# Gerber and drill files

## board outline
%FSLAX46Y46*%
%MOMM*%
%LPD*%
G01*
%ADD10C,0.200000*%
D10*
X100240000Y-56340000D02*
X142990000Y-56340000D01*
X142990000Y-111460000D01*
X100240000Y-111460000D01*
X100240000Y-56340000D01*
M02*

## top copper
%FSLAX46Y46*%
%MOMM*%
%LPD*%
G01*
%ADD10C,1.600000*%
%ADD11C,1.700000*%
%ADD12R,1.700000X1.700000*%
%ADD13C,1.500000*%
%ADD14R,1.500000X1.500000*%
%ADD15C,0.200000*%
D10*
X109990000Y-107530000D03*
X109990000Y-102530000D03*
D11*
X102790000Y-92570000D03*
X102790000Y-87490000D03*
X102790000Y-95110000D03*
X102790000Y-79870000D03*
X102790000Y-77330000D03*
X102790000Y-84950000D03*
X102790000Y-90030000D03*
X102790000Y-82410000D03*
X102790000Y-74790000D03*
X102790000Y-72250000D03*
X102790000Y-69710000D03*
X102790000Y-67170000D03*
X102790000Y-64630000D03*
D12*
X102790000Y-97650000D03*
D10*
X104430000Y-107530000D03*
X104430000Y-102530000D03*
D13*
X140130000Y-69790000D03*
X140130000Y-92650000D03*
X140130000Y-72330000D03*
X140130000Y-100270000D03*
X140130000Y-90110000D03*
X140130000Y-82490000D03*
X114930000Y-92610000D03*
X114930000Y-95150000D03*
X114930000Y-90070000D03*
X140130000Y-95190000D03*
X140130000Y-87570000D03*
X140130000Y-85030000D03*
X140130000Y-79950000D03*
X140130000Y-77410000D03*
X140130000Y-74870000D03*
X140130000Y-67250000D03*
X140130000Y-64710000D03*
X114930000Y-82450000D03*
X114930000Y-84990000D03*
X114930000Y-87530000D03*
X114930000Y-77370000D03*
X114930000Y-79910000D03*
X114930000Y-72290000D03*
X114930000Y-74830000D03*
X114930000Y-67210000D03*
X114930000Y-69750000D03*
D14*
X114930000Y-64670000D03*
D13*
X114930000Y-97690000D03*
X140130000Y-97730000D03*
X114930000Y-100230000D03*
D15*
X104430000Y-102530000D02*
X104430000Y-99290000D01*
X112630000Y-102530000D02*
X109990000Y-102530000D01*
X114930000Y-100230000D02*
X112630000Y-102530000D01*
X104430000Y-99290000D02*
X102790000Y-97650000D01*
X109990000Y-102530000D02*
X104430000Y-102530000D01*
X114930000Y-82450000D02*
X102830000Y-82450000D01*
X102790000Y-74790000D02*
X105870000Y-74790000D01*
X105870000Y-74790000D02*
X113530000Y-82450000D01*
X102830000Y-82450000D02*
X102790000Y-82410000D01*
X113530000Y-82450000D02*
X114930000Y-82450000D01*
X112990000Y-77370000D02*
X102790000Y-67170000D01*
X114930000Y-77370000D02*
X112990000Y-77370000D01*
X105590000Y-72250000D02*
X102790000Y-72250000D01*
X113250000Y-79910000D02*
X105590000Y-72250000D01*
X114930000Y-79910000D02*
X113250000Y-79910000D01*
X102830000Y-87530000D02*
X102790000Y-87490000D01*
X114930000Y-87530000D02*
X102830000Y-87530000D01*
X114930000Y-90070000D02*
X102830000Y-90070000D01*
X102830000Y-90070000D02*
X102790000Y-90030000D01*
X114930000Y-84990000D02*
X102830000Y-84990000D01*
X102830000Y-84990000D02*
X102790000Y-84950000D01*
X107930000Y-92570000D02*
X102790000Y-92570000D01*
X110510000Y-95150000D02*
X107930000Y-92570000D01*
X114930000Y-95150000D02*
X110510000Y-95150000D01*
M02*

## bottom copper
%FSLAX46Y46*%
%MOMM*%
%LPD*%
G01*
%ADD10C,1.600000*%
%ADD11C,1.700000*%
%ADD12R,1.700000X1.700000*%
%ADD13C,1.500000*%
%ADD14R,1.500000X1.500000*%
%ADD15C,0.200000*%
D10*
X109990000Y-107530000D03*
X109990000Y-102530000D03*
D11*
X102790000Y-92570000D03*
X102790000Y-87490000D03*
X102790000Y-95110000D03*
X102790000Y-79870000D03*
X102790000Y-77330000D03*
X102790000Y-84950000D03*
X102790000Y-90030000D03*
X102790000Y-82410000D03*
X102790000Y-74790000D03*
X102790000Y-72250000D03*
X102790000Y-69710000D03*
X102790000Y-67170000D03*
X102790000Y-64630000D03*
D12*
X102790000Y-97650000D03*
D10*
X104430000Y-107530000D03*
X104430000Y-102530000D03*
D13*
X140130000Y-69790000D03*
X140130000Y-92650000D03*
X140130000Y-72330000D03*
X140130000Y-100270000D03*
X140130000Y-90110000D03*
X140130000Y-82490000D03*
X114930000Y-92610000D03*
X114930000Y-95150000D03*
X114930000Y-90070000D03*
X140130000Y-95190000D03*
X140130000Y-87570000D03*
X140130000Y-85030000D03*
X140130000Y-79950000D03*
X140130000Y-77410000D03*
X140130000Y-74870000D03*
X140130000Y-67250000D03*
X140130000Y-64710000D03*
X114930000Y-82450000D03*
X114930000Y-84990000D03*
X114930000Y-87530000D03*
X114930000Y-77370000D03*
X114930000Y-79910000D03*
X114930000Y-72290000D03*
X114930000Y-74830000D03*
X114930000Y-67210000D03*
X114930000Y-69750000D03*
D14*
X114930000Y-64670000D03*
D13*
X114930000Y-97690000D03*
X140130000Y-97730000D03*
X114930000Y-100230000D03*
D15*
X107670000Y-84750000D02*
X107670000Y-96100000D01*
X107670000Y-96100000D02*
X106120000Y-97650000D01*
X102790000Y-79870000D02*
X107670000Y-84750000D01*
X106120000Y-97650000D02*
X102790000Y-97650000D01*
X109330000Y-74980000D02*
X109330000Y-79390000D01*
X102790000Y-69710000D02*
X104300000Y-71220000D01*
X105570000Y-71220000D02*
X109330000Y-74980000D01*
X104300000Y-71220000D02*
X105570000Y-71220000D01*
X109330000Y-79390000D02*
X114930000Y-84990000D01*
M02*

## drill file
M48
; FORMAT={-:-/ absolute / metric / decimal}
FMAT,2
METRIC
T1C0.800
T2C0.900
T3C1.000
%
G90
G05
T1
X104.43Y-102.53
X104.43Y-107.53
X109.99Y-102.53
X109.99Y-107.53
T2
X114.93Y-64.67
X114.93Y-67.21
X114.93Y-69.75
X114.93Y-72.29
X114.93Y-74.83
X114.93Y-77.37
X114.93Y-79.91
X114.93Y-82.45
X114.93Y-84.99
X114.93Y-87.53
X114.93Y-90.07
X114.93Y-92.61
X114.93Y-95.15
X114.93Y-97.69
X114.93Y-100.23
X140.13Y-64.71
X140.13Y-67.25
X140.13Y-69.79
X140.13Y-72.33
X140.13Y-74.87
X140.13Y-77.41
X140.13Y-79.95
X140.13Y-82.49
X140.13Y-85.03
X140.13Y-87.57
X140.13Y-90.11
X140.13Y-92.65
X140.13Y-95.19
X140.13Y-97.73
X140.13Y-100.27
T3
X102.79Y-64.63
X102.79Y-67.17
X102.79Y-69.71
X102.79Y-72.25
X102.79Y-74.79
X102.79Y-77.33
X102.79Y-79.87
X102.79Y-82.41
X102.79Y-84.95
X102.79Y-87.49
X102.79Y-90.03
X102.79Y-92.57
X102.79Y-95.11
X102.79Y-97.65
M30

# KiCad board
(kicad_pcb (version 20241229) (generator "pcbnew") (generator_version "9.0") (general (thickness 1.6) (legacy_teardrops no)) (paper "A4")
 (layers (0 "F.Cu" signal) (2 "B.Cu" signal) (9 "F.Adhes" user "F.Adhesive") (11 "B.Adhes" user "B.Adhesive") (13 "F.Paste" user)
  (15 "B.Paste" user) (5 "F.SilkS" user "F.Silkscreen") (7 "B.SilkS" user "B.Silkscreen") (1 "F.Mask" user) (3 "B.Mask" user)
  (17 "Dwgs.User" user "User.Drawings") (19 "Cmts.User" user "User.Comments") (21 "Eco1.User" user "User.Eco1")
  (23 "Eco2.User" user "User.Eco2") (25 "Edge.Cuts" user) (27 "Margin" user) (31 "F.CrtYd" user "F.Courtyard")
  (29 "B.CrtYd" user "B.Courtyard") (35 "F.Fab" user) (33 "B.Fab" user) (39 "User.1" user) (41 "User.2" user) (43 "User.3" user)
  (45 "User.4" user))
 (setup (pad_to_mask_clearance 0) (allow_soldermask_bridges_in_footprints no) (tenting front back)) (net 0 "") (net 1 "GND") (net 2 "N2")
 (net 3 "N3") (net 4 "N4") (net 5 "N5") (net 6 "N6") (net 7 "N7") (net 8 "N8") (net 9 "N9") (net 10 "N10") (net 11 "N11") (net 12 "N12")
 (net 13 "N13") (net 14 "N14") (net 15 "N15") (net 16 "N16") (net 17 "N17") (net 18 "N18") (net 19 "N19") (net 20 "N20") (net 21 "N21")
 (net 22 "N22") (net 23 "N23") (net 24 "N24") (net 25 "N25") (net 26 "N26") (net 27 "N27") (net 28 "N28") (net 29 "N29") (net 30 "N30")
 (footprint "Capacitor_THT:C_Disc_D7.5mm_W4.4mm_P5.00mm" (layer "F.Cu") (at 109.99 107.53 90)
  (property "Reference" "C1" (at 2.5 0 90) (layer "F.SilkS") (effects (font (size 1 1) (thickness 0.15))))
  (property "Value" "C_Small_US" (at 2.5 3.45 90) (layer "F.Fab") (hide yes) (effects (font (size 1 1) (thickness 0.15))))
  (pad "1" thru_hole circle (at 0 0 90) (size 1.6 1.6) (drill 0.8) (layers "*.Cu" "*.Mask") (remove_unused_layers no) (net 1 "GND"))
  (pad "2" thru_hole circle (at 5 0 90) (size 1.6 1.6) (drill 0.8) (layers "*.Cu" "*.Mask") (remove_unused_layers no) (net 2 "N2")))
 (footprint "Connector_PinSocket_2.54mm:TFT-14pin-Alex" (layer "F.Cu") (at 102.79 97.65 180)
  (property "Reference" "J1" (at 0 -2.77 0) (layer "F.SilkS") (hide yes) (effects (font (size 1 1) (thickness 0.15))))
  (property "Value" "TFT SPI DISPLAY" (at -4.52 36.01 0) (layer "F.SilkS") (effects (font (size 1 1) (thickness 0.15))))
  (pad "CS" thru_hole circle (at 0 5.08 180) (size 1.7 1.7) (drill 1) (layers "*.Cu" "*.Mask") (remove_unused_layers no) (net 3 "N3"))
  (pad "DC" thru_hole circle (at 0 10.16 180) (size 1.7 1.7) (drill 1) (layers "*.Cu" "*.Mask") (remove_unused_layers no) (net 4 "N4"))
  (pad "GND" thru_hole circle (at 0 2.54 180) (size 1.7 1.7) (drill 1) (layers "*.Cu" "*.Mask") (remove_unused_layers no) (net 1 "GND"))
  (pad "LED" thru_hole circle (at 0 17.78 180) (size 1.7 1.7) (drill 1) (layers "*.Cu" "*.Mask") (remove_unused_layers no) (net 2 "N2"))
  (pad "MISO" thru_hole circle (at 0 20.32 180) (size 1.7 1.7) (drill 1) (layers "*.Cu" "*.Mask") (remove_unused_layers no) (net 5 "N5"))
  (pad "MOSI" thru_hole circle (at 0 12.7 180) (size 1.7 1.7) (drill 1) (layers "*.Cu" "*.Mask") (remove_unused_layers no) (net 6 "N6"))
  (pad "RST" thru_hole circle (at 0 7.62 180) (size 1.7 1.7) (drill 1) (layers "*.Cu" "*.Mask") (remove_unused_layers no) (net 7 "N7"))
  (pad "SCK" thru_hole circle (at 0 15.24 180) (size 1.7 1.7) (drill 1) (layers "*.Cu" "*.Mask") (remove_unused_layers no) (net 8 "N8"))
  (pad "T_CLK" thru_hole circle (at 0 22.86 180) (size 1.7 1.7) (drill 1) (layers "*.Cu" "*.Mask") (remove_unused_layers no) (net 8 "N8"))
  (pad "T_CS" thru_hole circle (at 0 25.4 180) (size 1.7 1.7) (drill 1) (layers "*.Cu" "*.Mask") (remove_unused_layers no) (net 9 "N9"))
  (pad "T_DIN" thru_hole circle (at 0 27.94 180) (size 1.7 1.7) (drill 1) (layers "*.Cu" "*.Mask") (remove_unused_layers no) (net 6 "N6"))
  (pad "T_DO" thru_hole circle (at 0 30.48 180) (size 1.7 1.7) (drill 1) (layers "*.Cu" "*.Mask") (remove_unused_layers no) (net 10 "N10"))
  (pad "T_IRQ" thru_hole circle (at 0 33.02 180) (size 1.7 1.7) (drill 1) (layers "*.Cu" "*.Mask") (remove_unused_layers no) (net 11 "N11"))
  (pad "VCC" thru_hole rect (at 0 0 180) (size 1.7 1.7) (drill 1) (layers "*.Cu" "*.Mask") (remove_unused_layers no) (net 2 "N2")))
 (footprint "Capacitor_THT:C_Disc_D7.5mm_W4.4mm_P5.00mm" (layer "F.Cu") (at 104.43 107.53 90)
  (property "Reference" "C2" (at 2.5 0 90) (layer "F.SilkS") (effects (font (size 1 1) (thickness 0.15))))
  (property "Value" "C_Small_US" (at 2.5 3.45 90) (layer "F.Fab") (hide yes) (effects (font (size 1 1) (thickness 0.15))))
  (pad "1" thru_hole circle (at 0 0 90) (size 1.6 1.6) (drill 0.8) (layers "*.Cu" "*.Mask") (remove_unused_layers no) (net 1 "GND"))
  (pad "2" thru_hole circle (at 5 0 90) (size 1.6 1.6) (drill 0.8) (layers "*.Cu" "*.Mask") (remove_unused_layers no) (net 2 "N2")))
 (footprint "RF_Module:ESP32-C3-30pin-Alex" (layer "F.Cu") (at 114.93 64.67)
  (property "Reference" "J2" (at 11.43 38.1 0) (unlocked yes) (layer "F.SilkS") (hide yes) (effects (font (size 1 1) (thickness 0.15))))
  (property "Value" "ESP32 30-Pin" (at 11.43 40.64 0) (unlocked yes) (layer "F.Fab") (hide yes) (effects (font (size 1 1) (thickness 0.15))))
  (pad "1" thru_hole circle (at 25.2 5.12) (size 1.5 1.5) (drill 0.9) (layers "*.Cu" "*.Mask") (remove_unused_layers yes)
   (keep_end_layers yes) (zone_layer_connections) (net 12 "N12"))
  (pad "2" thru_hole circle (at 25.2 27.98) (size 1.5 1.5) (drill 0.9) (layers "*.Cu" "*.Mask") (remove_unused_layers yes)
   (keep_end_layers yes) (zone_layer_connections) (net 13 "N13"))
  (pad "3" thru_hole circle (at 25.2 7.66) (size 1.5 1.5) (drill 0.9) (layers "*.Cu" "*.Mask") (remove_unused_layers yes)
   (keep_end_layers yes) (zone_layer_connections) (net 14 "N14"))
  (pad "3.3V" thru_hole circle (at 25.2 35.6) (size 1.5 1.5) (drill 0.9) (layers "*.Cu" "*.Mask") (remove_unused_layers yes)
   (keep_end_layers yes) (zone_layer_connections))
  (pad "4" thru_hole circle (at 25.2 25.44) (size 1.5 1.5) (drill 0.9) (layers "*.Cu" "*.Mask") (remove_unused_layers yes)
   (keep_end_layers yes) (zone_layer_connections) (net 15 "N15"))
  (pad "5" thru_hole circle (at 25.2 17.82) (size 1.5 1.5) (drill 0.9) (layers "*.Cu" "*.Mask") (remove_unused_layers yes)
   (keep_end_layers yes) (zone_layer_connections) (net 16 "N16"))
  (pad "12" thru_hole circle (at 0 27.94) (size 1.5 1.5) (drill 0.9) (layers "*.Cu" "*.Mask") (remove_unused_layers yes)
   (keep_end_layers yes) (zone_layer_connections) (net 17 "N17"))
  (pad "13" thru_hole circle (at 0 30.48) (size 1.5 1.5) (drill 0.9) (layers "*.Cu" "*.Mask") (remove_unused_layers yes)
   (keep_end_layers yes) (zone_layer_connections) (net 3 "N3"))
  (pad "14" thru_hole circle (at 0 25.4) (size 1.5 1.5) (drill 0.9) (layers "*.Cu" "*.Mask") (remove_unused_layers yes)
   (keep_end_layers yes) (zone_layer_connections) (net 7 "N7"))
  (pad "15" thru_hole circle (at 25.2 30.52) (size 1.5 1.5) (drill 0.9) (layers "*.Cu" "*.Mask") (remove_unused_layers yes)
   (keep_end_layers yes) (zone_layer_connections) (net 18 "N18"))
  (pad "16" thru_hole circle (at 25.2 22.9) (size 1.5 1.5) (drill 0.9) (layers "*.Cu" "*.Mask") (remove_unused_layers yes)
   (keep_end_layers yes) (zone_layer_connections) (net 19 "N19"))
  (pad "17" thru_hole circle (at 25.2 20.36) (size 1.5 1.5) (drill 0.9) (layers "*.Cu" "*.Mask") (remove_unused_layers yes)
   (keep_end_layers yes) (zone_layer_connections) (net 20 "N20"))
  (pad "18" thru_hole circle (at 25.2 15.28) (size 1.5 1.5) (drill 0.9) (layers "*.Cu" "*.Mask") (remove_unused_layers yes)
   (keep_end_layers yes) (zone_layer_connections) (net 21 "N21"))
  (pad "19" thru_hole circle (at 25.2 12.74) (size 1.5 1.5) (drill 0.9) (layers "*.Cu" "*.Mask") (remove_unused_layers yes)
   (keep_end_layers yes) (zone_layer_connections) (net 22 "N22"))
  (pad "21" thru_hole circle (at 25.2 10.2) (size 1.5 1.5) (drill 0.9) (layers "*.Cu" "*.Mask") (remove_unused_layers yes)
   (keep_end_layers yes) (zone_layer_connections) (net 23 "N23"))
  (pad "22" thru_hole circle (at 25.2 2.58) (size 1.5 1.5) (drill 0.9) (layers "*.Cu" "*.Mask") (remove_unused_layers yes)
   (keep_end_layers yes) (zone_layer_connections) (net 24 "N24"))
  (pad "23" thru_hole circle (at 25.2 0.04) (size 1.5 1.5) (drill 0.9) (layers "*.Cu" "*.Mask") (remove_unused_layers yes)
   (keep_end_layers yes) (zone_layer_connections) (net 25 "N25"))
  (pad "25" thru_hole circle (at 0 17.78) (size 1.5 1.5) (drill 0.9) (layers "*.Cu" "*.Mask") (remove_unused_layers yes)
   (keep_end_layers yes) (zone_layer_connections) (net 8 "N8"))
  (pad "26" thru_hole circle (at 0 20.32) (size 1.5 1.5) (drill 0.9) (layers "*.Cu" "*.Mask") (remove_unused_layers yes)
   (keep_end_layers yes) (zone_layer_connections) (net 6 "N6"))
  (pad "27" thru_hole circle (at 0 22.86) (size 1.5 1.5) (drill 0.9) (layers "*.Cu" "*.Mask") (remove_unused_layers yes)
   (keep_end_layers yes) (zone_layer_connections) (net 4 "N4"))
  (pad "32" thru_hole circle (at 0 12.7) (size 1.5 1.5) (drill 0.9) (layers "*.Cu" "*.Mask") (remove_unused_layers yes)
   (keep_end_layers yes) (zone_layer_connections) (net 10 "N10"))
  (pad "33" thru_hole circle (at 0 15.24) (size 1.5 1.5) (drill 0.9) (layers "*.Cu" "*.Mask") (remove_unused_layers yes)
   (keep_end_layers yes) (zone_layer_connections) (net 9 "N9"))
  (pad "34" thru_hole circle (at 0 7.62) (size 1.5 1.5) (drill 0.9) (layers "*.Cu" "*.Mask") (remove_unused_layers yes)
   (keep_end_layers yes) (zone_layer_connections) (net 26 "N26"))
  (pad "35" thru_hole circle (at 0 10.16) (size 1.5 1.5) (drill 0.9) (layers "*.Cu" "*.Mask") (remove_unused_layers yes)
   (keep_end_layers yes) (zone_layer_connections) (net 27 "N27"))
  (pad "36" thru_hole circle (at 0 2.54) (size 1.5 1.5) (drill 0.9) (layers "*.Cu" "*.Mask") (remove_unused_layers yes)
   (keep_end_layers yes) (zone_layer_connections) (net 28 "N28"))
  (pad "39" thru_hole circle (at 0 5.08) (size 1.5 1.5) (drill 0.9) (layers "*.Cu" "*.Mask") (remove_unused_layers yes)
   (keep_end_layers yes) (zone_layer_connections) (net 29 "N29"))
  (pad "EN" thru_hole rect (at 0 0) (size 1.5 1.5) (drill 0.9) (layers "*.Cu" "*.Mask") (remove_unused_layers yes) (keep_end_layers yes)
   (zone_layer_connections) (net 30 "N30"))
  (pad "GND" thru_hole circle (at 0 33.02) (size 1.5 1.5) (drill 0.9) (layers "*.Cu" "*.Mask") (remove_unused_layers yes)
   (keep_end_layers yes) (zone_layer_connections) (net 1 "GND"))
  (pad "GND" thru_hole circle (at 25.2 33.06) (size 1.5 1.5) (drill 0.9) (layers "*.Cu" "*.Mask") (remove_unused_layers yes)
   (keep_end_layers yes) (zone_layer_connections) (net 1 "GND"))
  (pad "VIN" thru_hole circle (at 0 35.56) (size 1.5 1.5) (drill 0.9) (layers "*.Cu" "*.Mask") (remove_unused_layers yes)
   (keep_end_layers yes) (zone_layer_connections) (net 2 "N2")))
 (gr_rect (start 100.24 56.34) (end 142.99 111.46) (stroke (width 0.2) (type solid)) (fill no) (layer "Edge.Cuts"))
 (segment (start 104.43 102.53) (end 104.43 99.29) (width 0.2) (layer "F.Cu") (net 2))
 (segment (start 112.63 102.53) (end 109.99 102.53) (width 0.2) (layer "F.Cu") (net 2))
 (segment (start 114.93 100.23) (end 112.63 102.53) (width 0.2) (layer "F.Cu") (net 2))
 (segment (start 104.43 99.29) (end 102.79 97.65) (width 0.2) (layer "F.Cu") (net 2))
 (segment (start 109.99 102.53) (end 104.43 102.53) (width 0.2) (layer "F.Cu") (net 2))
 (segment (start 107.67 84.75) (end 107.67 96.1) (width 0.2) (layer "B.Cu") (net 2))
 (segment (start 107.67 96.1) (end 106.12 97.65) (width 0.2) (layer "B.Cu") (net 2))
 (segment (start 102.79 79.87) (end 107.67 84.75) (width 0.2) (layer "B.Cu") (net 2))
 (segment (start 106.12 97.65) (end 102.79 97.65) (width 0.2) (layer "B.Cu") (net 2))
 (segment (start 114.93 82.45) (end 102.83 82.45) (width 0.2) (layer "F.Cu") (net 8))
 (segment (start 102.79 74.79) (end 105.87 74.79) (width 0.2) (layer "F.Cu") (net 8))
 (segment (start 105.87 74.79) (end 113.53 82.45) (width 0.2) (layer "F.Cu") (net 8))
 (segment (start 102.83 82.45) (end 102.79 82.41) (width 0.2) (layer "F.Cu") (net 8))
 (segment (start 113.53 82.45) (end 114.93 82.45) (width 0.2) (layer "F.Cu") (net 8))
 (segment (start 112.99 77.37) (end 102.79 67.17) (width 0.2) (layer "F.Cu") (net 10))
 (segment (start 114.93 77.37) (end 112.99 77.37) (width 0.2) (layer "F.Cu") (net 10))
 (segment (start 105.59 72.25) (end 102.79 72.25) (width 0.2) (layer "F.Cu") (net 9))
 (segment (start 113.25 79.91) (end 105.59 72.25) (width 0.2) (layer "F.Cu") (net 9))
 (segment (start 114.93 79.91) (end 113.25 79.91) (width 0.2) (layer "F.Cu") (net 9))
 (segment (start 102.83 87.53) (end 102.79 87.49) (width 0.2) (layer "F.Cu") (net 4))
 (segment (start 114.93 87.53) (end 102.83 87.53) (width 0.2) (layer "F.Cu") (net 4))
 (segment (start 114.93 90.07) (end 102.83 90.07) (width 0.2) (layer "F.Cu") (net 7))
 (segment (start 102.83 90.07) (end 102.79 90.03) (width 0.2) (layer "F.Cu") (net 7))
 (segment (start 114.93 84.99) (end 102.83 84.99) (width 0.2) (layer "F.Cu") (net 6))
 (segment (start 102.83 84.99) (end 102.79 84.95) (width 0.2) (layer "F.Cu") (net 6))
 (segment (start 109.33 74.98) (end 109.33 79.39) (width 0.2) (layer "B.Cu") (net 6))
 (segment (start 102.79 69.71) (end 104.3 71.22) (width 0.2) (layer "B.Cu") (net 6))
 (segment (start 105.57 71.22) (end 109.33 74.98) (width 0.2) (layer "B.Cu") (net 6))
 (segment (start 104.3 71.22) (end 105.57 71.22) (width 0.2) (layer "B.Cu") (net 6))
 (segment (start 109.33 79.39) (end 114.93 84.99) (width 0.2) (layer "B.Cu") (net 6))
 (segment (start 107.93 92.57) (end 102.79 92.57) (width 0.2) (layer "F.Cu") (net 3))
 (segment (start 110.51 95.15) (end 107.93 92.57) (width 0.2) (layer "F.Cu") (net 3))
 (segment (start 114.93 95.15) (end 110.51 95.15) (width 0.2) (layer "F.Cu") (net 3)))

